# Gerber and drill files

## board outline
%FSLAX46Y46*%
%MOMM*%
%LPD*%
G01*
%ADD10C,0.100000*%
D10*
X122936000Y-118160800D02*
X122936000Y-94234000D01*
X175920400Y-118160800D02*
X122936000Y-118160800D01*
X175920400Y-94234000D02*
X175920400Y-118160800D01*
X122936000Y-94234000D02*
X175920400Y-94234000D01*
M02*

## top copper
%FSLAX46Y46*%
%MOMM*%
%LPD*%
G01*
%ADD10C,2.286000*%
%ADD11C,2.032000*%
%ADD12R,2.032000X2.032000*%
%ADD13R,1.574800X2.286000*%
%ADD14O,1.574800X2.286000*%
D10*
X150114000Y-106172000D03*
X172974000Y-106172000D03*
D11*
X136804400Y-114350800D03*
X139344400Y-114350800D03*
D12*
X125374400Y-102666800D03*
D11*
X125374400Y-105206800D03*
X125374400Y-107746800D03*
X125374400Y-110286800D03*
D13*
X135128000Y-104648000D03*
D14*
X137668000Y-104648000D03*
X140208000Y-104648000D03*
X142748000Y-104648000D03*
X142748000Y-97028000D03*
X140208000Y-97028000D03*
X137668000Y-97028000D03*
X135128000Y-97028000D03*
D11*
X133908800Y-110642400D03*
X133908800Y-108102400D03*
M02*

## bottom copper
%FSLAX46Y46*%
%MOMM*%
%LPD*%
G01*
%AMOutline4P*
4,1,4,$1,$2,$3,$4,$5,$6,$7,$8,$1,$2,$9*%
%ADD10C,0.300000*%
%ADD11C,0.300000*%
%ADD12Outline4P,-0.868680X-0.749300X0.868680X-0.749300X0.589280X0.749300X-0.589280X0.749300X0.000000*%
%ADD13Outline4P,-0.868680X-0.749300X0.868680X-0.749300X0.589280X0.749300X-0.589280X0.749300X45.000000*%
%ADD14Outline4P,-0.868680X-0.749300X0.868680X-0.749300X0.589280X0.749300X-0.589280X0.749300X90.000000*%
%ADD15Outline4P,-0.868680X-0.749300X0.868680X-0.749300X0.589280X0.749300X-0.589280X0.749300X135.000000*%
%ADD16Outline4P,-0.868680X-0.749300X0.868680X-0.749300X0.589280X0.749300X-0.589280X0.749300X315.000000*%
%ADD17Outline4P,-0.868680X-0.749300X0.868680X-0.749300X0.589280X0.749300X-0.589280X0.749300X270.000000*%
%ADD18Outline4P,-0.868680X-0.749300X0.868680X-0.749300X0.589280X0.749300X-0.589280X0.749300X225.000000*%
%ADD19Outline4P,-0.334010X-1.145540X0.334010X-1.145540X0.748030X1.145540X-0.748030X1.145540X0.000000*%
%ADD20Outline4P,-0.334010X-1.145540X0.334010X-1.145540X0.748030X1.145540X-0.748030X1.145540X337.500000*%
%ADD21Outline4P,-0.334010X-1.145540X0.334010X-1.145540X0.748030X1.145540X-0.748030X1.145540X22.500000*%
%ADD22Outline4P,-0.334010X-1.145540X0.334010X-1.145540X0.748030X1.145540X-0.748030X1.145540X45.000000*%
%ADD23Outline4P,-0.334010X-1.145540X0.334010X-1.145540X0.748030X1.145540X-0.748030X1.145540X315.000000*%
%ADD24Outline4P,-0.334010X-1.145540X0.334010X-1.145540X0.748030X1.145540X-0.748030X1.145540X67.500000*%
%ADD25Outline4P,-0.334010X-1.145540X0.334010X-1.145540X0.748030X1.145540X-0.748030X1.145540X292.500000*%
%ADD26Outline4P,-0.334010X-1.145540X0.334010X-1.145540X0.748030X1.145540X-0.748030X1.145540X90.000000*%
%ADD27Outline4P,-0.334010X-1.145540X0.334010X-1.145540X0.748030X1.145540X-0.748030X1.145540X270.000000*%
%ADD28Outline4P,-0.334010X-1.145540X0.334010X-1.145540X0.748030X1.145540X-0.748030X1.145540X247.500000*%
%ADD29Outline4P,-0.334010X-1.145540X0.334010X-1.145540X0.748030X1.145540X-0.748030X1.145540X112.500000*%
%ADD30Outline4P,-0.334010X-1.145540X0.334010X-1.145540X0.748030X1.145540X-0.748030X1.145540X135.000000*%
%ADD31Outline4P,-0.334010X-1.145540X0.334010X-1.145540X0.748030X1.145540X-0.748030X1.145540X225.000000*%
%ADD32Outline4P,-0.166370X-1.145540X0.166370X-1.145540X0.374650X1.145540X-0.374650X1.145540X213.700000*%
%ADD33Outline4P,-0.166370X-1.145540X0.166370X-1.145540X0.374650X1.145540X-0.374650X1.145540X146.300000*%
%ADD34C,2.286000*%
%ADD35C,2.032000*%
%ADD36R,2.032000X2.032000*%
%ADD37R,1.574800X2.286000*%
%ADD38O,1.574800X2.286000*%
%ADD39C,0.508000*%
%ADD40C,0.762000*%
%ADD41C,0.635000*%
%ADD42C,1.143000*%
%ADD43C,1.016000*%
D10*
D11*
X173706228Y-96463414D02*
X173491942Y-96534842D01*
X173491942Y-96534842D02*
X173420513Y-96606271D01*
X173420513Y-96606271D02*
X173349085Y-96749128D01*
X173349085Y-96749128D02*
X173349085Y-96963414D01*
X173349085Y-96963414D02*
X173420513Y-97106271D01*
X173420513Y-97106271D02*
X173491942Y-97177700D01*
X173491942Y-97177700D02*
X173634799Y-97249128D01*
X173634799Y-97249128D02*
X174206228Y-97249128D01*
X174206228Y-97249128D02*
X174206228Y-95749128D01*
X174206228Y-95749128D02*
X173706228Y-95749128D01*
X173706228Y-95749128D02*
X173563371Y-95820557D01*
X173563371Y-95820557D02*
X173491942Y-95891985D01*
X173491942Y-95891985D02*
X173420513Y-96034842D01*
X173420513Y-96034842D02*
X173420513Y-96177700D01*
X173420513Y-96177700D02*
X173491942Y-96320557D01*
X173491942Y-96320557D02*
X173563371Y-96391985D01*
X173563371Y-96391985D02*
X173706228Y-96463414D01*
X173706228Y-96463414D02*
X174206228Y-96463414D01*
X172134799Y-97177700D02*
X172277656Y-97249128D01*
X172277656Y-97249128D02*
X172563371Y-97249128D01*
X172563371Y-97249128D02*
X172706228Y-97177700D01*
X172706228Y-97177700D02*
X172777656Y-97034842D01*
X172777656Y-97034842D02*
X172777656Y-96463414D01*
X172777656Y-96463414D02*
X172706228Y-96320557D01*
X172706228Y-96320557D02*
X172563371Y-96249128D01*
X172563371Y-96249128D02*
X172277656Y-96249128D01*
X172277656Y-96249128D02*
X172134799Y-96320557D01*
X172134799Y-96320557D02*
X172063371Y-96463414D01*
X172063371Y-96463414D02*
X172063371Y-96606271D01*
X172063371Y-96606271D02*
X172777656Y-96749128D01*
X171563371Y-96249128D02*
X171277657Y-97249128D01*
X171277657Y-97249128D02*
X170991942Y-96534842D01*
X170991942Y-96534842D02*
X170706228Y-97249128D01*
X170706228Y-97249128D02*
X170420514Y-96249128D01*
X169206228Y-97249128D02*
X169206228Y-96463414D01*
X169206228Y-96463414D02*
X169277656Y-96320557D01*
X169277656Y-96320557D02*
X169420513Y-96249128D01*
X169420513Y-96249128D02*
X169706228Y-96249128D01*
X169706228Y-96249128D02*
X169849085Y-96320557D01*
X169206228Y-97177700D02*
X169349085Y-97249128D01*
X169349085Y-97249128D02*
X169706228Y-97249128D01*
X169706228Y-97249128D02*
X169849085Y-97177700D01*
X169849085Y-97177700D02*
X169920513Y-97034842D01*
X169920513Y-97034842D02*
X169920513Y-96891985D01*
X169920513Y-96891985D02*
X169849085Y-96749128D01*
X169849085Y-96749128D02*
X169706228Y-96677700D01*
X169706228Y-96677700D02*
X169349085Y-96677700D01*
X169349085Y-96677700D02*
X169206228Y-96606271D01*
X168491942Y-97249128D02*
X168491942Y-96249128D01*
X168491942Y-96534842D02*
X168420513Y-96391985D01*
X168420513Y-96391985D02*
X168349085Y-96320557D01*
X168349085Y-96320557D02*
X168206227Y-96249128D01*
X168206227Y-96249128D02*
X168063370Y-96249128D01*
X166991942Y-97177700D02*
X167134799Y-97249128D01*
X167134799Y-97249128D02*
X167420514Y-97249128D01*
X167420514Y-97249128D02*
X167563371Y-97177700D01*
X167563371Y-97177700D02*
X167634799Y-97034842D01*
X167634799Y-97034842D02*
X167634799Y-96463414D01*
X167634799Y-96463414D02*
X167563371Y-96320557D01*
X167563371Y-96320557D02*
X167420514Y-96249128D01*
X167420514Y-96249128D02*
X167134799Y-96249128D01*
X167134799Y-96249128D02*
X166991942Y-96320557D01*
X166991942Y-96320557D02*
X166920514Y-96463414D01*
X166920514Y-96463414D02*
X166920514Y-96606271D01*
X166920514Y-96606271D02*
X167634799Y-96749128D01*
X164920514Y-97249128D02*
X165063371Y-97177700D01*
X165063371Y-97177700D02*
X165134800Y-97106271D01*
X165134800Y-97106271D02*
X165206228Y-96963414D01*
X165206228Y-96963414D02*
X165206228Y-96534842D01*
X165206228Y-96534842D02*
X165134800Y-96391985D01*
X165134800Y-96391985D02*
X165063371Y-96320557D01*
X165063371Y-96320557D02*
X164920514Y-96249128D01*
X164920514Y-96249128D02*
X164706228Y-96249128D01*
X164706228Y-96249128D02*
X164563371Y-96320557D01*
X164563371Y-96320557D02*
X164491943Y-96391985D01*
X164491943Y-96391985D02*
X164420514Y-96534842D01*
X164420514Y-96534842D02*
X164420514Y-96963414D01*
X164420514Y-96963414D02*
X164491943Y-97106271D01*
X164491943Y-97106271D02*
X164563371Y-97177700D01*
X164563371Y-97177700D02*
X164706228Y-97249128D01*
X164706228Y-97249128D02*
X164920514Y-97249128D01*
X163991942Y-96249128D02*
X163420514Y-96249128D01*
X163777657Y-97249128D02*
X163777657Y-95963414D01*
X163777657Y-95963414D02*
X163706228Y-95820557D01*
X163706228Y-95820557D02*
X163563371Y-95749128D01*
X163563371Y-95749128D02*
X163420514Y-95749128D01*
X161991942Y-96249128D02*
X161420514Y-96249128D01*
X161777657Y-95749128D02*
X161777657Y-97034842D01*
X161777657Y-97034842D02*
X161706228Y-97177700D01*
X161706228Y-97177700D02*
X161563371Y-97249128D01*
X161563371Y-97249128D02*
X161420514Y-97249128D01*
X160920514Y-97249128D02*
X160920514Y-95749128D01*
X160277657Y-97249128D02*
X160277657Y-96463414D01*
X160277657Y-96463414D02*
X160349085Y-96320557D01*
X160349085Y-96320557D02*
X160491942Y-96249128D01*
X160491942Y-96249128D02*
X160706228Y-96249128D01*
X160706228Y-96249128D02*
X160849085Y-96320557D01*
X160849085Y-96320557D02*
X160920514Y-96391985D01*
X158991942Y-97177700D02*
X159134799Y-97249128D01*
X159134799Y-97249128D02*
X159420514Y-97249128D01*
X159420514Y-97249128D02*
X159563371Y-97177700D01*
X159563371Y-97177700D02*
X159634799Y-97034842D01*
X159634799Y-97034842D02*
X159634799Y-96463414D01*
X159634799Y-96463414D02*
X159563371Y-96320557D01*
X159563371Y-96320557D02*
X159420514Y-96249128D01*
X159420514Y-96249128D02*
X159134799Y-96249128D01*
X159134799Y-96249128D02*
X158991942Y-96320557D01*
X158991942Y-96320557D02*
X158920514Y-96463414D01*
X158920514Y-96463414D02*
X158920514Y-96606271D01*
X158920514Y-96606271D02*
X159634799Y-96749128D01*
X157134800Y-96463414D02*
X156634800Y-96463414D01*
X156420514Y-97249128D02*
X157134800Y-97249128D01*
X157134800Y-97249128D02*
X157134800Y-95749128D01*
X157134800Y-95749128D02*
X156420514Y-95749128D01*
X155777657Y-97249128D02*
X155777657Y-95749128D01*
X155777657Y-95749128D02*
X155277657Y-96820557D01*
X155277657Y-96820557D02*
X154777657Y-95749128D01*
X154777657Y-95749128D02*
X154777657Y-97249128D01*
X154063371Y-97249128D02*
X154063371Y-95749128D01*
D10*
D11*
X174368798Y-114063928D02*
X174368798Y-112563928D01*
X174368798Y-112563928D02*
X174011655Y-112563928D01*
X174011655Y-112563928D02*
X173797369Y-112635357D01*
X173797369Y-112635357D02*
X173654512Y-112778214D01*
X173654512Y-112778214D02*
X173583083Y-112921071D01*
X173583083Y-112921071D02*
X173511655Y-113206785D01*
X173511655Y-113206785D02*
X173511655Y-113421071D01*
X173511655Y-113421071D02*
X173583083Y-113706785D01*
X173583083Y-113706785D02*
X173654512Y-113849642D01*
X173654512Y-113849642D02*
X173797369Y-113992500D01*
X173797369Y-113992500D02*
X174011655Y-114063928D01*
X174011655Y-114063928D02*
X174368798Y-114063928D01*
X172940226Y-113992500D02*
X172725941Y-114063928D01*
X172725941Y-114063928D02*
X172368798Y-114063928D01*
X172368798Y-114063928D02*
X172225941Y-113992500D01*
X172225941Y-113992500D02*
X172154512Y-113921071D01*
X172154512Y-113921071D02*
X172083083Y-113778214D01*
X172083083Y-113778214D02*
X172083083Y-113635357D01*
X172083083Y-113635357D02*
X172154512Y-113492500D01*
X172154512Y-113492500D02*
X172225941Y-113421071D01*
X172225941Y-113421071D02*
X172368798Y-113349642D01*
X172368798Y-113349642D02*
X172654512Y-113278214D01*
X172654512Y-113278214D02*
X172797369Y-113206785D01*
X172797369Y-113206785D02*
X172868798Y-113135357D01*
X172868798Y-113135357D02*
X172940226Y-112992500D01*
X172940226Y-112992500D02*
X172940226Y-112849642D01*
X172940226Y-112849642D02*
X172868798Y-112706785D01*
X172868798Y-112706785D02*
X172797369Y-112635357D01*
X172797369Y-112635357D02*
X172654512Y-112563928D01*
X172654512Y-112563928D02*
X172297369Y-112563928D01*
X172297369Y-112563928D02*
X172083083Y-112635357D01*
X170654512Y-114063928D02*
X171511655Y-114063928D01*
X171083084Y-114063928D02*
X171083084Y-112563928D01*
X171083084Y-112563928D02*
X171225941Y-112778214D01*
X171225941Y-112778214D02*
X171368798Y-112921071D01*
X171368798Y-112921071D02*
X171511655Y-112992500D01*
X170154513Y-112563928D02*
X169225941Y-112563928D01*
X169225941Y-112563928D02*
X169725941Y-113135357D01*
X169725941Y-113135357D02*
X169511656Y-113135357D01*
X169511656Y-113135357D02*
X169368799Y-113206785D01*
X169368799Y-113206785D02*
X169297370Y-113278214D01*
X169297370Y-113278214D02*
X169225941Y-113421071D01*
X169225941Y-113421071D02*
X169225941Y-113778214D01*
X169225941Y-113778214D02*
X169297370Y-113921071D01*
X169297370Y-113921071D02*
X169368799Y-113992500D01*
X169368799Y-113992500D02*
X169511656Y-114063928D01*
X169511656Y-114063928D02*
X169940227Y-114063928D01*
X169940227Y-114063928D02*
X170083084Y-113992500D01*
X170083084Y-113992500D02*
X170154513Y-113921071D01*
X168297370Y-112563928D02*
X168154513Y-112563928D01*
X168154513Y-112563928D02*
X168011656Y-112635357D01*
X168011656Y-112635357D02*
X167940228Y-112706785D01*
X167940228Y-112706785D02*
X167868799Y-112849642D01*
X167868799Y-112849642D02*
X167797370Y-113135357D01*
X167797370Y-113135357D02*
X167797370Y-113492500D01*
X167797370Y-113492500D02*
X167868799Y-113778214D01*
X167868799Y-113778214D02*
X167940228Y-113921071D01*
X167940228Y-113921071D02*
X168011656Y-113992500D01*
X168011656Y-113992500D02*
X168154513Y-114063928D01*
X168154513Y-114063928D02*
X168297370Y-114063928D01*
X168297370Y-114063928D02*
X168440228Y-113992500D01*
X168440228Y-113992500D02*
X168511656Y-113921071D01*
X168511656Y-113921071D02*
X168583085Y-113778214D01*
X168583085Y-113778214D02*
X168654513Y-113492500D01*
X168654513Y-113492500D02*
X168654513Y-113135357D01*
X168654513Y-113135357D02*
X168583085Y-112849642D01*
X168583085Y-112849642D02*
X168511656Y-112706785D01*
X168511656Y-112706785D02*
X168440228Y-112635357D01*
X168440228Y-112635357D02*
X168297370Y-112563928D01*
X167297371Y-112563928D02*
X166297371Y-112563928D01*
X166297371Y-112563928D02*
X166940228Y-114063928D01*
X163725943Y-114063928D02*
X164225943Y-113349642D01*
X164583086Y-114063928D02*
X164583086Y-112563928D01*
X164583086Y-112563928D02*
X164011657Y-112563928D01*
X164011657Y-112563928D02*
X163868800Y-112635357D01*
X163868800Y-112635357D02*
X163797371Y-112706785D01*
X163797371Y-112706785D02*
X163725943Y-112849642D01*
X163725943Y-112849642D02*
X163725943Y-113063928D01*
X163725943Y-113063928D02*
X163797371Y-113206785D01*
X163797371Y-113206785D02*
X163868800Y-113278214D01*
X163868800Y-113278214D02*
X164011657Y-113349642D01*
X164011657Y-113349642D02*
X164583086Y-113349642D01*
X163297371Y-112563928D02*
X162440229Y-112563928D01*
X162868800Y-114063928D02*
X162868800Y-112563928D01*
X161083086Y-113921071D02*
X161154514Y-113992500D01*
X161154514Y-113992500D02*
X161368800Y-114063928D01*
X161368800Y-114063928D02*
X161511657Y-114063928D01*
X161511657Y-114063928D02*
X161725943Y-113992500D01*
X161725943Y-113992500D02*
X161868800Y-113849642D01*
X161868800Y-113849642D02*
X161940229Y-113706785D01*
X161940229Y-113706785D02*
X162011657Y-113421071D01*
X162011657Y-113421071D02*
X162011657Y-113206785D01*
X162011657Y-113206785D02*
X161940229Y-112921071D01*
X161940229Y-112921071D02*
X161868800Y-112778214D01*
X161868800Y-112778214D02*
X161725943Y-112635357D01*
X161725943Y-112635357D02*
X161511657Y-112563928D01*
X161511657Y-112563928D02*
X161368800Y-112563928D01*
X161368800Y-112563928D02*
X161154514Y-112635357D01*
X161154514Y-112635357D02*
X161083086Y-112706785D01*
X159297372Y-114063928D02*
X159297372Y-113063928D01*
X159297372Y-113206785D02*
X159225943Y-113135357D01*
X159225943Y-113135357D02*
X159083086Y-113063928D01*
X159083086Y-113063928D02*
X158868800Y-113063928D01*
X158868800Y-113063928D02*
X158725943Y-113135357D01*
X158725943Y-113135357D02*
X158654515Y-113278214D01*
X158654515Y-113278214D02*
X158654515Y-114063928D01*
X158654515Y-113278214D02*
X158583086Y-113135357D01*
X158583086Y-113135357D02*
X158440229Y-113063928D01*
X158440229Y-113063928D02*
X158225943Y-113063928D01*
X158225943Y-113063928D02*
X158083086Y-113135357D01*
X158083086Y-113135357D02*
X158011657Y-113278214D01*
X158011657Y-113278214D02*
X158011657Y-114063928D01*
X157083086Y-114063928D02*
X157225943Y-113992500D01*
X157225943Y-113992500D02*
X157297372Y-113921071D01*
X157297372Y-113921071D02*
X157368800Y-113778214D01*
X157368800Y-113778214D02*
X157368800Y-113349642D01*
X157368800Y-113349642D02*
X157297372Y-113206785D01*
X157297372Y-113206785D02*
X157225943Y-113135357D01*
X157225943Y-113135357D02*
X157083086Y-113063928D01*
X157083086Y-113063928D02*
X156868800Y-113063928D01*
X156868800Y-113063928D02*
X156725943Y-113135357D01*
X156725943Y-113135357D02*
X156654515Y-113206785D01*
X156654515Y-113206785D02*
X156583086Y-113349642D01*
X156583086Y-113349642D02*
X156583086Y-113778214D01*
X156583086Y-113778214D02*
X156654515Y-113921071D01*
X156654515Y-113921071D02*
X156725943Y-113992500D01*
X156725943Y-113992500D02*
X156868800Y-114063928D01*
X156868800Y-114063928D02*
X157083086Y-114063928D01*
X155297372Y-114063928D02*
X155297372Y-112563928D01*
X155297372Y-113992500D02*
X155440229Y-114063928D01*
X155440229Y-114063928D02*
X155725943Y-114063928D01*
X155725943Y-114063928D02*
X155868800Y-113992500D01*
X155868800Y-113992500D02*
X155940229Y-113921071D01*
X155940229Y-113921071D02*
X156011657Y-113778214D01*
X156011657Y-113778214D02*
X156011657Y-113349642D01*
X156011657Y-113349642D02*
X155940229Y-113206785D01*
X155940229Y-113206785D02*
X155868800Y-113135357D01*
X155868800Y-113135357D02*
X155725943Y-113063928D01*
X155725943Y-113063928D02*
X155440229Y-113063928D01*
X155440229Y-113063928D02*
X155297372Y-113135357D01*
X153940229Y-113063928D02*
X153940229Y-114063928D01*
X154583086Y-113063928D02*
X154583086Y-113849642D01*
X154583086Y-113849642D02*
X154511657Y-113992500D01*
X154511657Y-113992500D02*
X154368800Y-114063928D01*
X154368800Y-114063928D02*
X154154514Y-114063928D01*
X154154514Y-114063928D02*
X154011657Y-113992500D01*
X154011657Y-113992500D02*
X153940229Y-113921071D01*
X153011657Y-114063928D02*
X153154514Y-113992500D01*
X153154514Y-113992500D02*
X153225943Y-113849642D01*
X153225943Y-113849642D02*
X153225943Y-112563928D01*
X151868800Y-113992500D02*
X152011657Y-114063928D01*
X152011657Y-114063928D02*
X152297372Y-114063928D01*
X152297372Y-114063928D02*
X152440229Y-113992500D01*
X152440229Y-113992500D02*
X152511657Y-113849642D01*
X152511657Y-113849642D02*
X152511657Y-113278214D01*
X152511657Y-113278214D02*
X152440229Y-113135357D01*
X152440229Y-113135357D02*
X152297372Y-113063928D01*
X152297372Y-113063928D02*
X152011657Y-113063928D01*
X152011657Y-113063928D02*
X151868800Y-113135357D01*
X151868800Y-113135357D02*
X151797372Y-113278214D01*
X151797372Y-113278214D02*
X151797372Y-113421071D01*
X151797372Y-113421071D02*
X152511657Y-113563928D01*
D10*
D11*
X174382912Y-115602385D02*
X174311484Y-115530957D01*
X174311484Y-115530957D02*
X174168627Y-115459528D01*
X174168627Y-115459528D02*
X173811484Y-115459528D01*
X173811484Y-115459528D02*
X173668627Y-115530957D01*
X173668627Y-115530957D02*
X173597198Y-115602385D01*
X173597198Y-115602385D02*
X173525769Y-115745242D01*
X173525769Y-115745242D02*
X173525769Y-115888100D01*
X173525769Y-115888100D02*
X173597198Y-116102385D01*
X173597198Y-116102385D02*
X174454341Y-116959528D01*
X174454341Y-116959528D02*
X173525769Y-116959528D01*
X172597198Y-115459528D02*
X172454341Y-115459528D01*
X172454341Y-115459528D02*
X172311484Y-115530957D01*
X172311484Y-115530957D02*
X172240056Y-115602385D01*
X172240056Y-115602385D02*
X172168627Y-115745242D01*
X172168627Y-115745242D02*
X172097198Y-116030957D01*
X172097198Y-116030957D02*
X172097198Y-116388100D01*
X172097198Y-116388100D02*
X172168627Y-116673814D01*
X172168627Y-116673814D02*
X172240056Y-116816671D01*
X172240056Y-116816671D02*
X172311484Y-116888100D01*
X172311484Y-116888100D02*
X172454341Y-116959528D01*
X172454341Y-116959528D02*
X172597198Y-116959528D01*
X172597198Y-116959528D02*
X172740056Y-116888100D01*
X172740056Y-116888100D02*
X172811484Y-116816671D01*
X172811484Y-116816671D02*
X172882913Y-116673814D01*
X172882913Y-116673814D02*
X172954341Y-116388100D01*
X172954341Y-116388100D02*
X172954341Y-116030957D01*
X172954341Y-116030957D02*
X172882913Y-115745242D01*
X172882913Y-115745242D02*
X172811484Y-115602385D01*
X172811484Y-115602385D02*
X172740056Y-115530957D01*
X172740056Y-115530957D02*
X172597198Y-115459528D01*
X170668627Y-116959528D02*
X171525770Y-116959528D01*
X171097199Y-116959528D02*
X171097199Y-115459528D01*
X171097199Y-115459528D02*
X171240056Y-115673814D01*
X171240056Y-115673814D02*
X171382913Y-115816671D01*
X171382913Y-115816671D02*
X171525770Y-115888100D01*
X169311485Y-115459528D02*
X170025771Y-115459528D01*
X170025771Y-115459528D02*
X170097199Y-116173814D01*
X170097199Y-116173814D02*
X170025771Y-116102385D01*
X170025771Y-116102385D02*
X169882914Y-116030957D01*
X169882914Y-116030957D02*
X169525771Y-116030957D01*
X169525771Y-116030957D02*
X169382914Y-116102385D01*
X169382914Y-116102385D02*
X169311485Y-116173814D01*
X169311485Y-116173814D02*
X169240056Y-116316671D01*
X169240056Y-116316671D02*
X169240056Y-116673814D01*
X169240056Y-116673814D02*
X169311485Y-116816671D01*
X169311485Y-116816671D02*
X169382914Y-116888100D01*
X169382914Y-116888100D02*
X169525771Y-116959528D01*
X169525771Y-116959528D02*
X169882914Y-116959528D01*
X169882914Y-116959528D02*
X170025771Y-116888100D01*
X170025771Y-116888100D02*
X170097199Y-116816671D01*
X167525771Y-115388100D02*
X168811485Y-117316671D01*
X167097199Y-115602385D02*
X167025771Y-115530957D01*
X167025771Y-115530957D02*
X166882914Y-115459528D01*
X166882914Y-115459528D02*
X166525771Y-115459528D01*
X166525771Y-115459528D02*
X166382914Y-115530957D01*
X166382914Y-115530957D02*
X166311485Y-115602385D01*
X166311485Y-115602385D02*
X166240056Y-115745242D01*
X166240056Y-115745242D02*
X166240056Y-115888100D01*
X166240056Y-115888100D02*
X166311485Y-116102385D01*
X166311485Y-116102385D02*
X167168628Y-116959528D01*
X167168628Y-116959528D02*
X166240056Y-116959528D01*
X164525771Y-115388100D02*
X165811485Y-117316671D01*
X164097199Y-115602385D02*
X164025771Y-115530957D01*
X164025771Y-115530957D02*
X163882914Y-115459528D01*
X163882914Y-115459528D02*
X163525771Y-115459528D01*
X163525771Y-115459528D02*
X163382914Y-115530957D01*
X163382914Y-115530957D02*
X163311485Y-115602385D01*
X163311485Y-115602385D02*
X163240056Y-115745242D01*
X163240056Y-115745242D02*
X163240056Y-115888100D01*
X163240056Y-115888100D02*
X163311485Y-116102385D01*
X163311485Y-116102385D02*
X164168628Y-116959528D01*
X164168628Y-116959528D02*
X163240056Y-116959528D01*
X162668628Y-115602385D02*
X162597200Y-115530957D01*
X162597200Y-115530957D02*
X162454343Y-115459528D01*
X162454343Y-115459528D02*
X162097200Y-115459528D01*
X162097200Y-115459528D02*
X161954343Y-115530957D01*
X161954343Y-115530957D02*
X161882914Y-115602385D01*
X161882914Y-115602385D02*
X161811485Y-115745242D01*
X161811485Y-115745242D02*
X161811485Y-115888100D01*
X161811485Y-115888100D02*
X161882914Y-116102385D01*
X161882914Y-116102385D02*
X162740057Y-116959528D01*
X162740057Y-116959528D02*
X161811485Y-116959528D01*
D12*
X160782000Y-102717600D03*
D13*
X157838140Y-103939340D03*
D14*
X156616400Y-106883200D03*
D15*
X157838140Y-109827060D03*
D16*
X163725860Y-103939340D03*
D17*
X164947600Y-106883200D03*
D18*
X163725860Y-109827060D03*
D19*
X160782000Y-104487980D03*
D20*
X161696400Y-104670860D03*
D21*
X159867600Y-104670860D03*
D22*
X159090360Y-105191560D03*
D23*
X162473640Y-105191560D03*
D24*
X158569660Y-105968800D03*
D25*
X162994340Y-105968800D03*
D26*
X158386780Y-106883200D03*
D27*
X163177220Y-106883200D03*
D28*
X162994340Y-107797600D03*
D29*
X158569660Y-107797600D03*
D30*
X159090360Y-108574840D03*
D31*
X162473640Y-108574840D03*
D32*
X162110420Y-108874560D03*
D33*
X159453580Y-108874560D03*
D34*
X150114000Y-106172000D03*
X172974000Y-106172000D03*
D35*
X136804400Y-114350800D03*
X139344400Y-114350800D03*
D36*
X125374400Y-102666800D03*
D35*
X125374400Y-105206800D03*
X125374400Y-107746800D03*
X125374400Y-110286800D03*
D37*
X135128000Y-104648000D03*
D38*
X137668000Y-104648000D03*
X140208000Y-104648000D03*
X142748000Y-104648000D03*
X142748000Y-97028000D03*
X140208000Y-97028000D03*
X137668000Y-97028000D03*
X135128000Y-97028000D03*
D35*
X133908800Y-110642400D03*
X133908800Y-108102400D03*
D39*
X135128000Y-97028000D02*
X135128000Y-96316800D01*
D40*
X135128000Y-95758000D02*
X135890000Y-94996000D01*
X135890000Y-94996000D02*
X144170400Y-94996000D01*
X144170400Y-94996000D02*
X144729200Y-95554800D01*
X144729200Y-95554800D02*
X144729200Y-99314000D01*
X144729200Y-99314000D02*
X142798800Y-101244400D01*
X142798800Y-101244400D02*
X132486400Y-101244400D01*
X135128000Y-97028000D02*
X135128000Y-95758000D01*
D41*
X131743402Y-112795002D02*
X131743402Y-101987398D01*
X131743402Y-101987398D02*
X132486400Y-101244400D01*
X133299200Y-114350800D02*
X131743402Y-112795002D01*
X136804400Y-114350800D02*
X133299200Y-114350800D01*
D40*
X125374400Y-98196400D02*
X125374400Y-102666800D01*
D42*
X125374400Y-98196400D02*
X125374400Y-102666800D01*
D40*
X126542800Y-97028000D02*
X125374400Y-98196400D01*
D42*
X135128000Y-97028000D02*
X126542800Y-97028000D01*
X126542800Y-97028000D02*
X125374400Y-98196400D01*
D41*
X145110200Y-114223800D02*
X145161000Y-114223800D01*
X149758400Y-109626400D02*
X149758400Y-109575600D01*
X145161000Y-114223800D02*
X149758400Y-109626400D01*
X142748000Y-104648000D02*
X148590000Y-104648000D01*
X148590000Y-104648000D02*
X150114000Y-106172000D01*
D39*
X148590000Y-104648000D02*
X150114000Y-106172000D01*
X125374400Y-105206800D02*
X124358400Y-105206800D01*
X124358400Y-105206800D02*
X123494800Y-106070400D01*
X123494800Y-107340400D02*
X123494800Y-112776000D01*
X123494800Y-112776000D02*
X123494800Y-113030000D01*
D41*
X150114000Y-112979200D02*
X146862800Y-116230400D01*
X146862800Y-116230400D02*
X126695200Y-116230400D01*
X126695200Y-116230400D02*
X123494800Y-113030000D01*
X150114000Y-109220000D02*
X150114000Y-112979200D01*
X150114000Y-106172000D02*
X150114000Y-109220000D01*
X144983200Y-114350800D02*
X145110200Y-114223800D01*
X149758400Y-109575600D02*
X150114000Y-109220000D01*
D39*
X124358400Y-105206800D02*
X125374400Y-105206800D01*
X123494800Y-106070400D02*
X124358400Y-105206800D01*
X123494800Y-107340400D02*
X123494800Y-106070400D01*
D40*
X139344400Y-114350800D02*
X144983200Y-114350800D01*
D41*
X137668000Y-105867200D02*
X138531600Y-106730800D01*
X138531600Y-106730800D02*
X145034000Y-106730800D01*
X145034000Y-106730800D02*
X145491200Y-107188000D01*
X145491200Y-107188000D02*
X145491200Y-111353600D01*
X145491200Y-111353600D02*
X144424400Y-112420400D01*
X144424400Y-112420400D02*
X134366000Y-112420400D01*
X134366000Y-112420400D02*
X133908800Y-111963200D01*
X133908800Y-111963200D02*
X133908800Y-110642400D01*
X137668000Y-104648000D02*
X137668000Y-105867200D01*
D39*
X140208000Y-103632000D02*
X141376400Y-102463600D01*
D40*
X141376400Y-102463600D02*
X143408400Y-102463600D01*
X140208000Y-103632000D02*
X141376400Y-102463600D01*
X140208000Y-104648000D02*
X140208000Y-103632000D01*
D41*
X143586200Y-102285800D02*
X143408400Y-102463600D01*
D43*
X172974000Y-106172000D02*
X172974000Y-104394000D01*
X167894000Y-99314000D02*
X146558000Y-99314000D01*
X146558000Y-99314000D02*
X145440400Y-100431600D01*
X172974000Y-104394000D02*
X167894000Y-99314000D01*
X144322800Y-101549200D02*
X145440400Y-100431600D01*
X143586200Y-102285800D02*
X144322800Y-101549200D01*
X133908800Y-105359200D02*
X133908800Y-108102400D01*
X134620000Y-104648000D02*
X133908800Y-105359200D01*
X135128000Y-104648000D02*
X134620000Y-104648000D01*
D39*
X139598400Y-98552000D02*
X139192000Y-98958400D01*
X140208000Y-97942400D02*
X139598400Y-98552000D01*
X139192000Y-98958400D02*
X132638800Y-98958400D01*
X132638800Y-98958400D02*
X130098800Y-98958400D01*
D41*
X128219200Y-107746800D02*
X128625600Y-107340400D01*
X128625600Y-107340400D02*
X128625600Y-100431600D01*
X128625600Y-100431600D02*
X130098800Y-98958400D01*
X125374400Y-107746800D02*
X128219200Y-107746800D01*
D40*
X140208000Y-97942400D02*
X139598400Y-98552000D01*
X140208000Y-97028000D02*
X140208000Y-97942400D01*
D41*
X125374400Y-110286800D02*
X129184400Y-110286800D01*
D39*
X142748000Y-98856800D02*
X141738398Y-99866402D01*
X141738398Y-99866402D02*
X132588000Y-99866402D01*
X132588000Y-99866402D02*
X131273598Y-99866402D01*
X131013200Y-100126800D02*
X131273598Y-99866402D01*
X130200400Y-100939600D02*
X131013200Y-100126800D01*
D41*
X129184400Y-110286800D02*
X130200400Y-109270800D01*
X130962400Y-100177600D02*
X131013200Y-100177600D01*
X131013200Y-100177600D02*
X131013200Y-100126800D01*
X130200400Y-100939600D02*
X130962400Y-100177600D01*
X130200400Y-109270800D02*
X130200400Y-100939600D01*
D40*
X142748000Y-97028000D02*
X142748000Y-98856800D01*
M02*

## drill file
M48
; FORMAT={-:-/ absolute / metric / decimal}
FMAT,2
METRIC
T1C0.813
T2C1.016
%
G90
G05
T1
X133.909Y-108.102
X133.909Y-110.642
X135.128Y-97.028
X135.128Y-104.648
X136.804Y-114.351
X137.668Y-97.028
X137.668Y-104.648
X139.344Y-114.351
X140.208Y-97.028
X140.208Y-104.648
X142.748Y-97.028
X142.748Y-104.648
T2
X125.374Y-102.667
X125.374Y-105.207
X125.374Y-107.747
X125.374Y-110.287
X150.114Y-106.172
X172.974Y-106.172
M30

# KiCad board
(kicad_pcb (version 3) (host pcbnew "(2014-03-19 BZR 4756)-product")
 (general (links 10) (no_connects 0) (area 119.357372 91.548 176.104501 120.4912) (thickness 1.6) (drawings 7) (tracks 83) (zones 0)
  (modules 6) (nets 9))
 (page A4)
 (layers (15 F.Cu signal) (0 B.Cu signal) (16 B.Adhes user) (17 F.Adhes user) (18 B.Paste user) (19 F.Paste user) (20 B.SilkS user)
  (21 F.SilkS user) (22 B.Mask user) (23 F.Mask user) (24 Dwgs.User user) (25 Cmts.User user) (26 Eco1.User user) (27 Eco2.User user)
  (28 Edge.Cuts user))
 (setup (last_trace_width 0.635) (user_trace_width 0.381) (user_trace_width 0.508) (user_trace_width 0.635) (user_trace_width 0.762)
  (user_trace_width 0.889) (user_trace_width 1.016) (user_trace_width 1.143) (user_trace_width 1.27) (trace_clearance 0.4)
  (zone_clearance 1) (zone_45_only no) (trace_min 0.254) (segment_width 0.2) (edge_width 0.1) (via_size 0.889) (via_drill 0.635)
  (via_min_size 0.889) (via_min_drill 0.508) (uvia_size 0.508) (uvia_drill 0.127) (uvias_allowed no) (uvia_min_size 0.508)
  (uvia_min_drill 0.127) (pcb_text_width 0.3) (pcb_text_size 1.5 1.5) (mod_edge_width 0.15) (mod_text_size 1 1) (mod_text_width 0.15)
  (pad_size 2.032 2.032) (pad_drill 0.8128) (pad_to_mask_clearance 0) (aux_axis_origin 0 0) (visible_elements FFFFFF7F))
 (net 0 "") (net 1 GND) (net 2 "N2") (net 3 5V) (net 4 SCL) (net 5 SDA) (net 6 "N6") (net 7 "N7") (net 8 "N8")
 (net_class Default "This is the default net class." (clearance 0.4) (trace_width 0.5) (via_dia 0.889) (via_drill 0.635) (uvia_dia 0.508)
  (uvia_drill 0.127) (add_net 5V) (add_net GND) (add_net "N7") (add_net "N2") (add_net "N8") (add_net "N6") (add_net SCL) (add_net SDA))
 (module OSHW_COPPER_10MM (layer B.Cu) (at 160.782 106.8832 180)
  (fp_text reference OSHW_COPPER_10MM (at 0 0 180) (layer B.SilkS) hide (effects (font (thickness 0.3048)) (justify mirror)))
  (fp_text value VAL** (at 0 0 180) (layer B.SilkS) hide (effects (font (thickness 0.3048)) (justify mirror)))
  (pad "" smd trapezoid (at 0 4.1656) (size 1.45796 1.4986) (rect_delta 0 0.2794) (layers B.Cu B.Paste B.Mask))
  (pad "" smd trapezoid (at 2.94386 2.94386 45) (size 1.45796 1.4986) (rect_delta 0 0.2794) (layers B.Cu B.Paste B.Mask))
  (pad "" smd trapezoid (at 4.1656 0 90) (size 1.45796 1.4986) (rect_delta 0 0.2794) (layers B.Cu B.Paste B.Mask))
  (pad "" smd trapezoid (at 2.94386 -2.94386 135) (size 1.45796 1.4986) (rect_delta 0 0.2794) (layers B.Cu B.Paste B.Mask))
  (pad "" smd trapezoid (at -2.94386 2.94386 315) (size 1.45796 1.4986) (rect_delta 0 0.2794) (layers B.Cu B.Paste B.Mask))
  (pad "" smd trapezoid (at -4.1656 0 270) (size 1.45796 1.4986) (rect_delta 0 0.2794) (layers B.Cu B.Paste B.Mask))
  (pad "" smd trapezoid (at -2.94386 -2.94386 225) (size 1.45796 1.4986) (rect_delta 0 0.2794) (layers B.Cu B.Paste B.Mask))
  (pad "" smd trapezoid (at 0 2.39522) (size 1.08204 2.29108) (rect_delta 0 -0.41402) (layers B.Cu B.Paste B.Mask))
  (pad "" smd trapezoid (at -0.9144 2.21234 337.5) (size 1.08204 2.29108) (rect_delta 0 -0.41402) (layers B.Cu B.Paste B.Mask))
  (pad "" smd trapezoid (at 0.9144 2.21234 22.5) (size 1.08204 2.29108) (rect_delta 0 -0.41402) (layers B.Cu B.Paste B.Mask))
  (pad "" smd trapezoid (at 1.69164 1.69164 45) (size 1.08204 2.29108) (rect_delta 0 -0.41402) (layers B.Cu B.Paste B.Mask))
  (pad "" smd trapezoid (at -1.69164 1.69164 315) (size 1.08204 2.29108) (rect_delta 0 -0.41402) (layers B.Cu B.Paste B.Mask))
  (pad "" smd trapezoid (at 2.21234 0.9144 67.5) (size 1.08204 2.29108) (rect_delta 0 -0.41402) (layers B.Cu B.Paste B.Mask))
  (pad "" smd trapezoid (at -2.21234 0.9144 292.5) (size 1.08204 2.29108) (rect_delta 0 -0.41402) (layers B.Cu B.Paste B.Mask))
  (pad "" smd trapezoid (at 2.39522 0 90) (size 1.08204 2.29108) (rect_delta 0 -0.41402) (layers B.Cu B.Paste B.Mask))
  (pad "" smd trapezoid (at -2.39522 0 270) (size 1.08204 2.29108) (rect_delta 0 -0.41402) (layers B.Cu B.Paste B.Mask))
  (pad "" smd trapezoid (at -2.21234 -0.9144 247.5) (size 1.08204 2.29108) (rect_delta 0 -0.41402) (layers B.Cu B.Paste B.Mask))
  (pad "" smd trapezoid (at 2.21234 -0.9144 112.5) (size 1.08204 2.29108) (rect_delta 0 -0.41402) (layers B.Cu B.Paste B.Mask))
  (pad "" smd trapezoid (at 1.69164 -1.69164 135) (size 1.08204 2.29108) (rect_delta 0 -0.41402) (layers B.Cu B.Paste B.Mask))
  (pad "" smd trapezoid (at -1.69164 -1.69164 225) (size 1.08204 2.29108) (rect_delta 0 -0.41402) (layers B.Cu B.Paste B.Mask))
  (pad "" smd trapezoid (at -1.32842 -1.99136 213.7) (size 0.54102 2.29108) (rect_delta 0 -0.20828) (layers B.Cu B.Paste B.Mask))
  (pad "" smd trapezoid (at 1.32842 -1.99136 146.3) (size 0.54102 2.29108) (rect_delta 0 -0.20828) (layers B.Cu B.Paste B.Mask)))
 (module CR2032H (layer F.Cu) (at 157.734 106.172)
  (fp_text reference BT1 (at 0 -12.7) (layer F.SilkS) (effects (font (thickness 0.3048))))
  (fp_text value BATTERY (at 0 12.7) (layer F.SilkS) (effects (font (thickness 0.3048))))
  (pad 2 thru_hole circle (at -7.62 0) (size 2.286 2.286) (drill 1.016) (layers *.Cu *.Mask F.SilkS) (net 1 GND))
  (pad 1 thru_hole circle (at 15.24 0) (size 2.286 2.286) (drill 1.016) (layers *.Cu *.Mask F.SilkS) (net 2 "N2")))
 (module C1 (layer F.Cu) (at 138.0744 114.3508)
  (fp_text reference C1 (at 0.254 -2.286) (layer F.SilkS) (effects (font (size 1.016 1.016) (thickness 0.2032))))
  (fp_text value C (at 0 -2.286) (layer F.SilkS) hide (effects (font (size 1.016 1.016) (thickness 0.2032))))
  (pad 1 thru_hole circle (at -1.27 0) (size 2.032 2.032) (drill 0.8128) (layers *.Cu *.Mask F.SilkS) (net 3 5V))
  (pad 2 thru_hole circle (at 1.27 0) (size 2.032 2.032) (drill 0.8128) (layers *.Cu *.Mask F.SilkS) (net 1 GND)))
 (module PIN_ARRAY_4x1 (layer F.Cu) (at 125.3744 106.4768 270)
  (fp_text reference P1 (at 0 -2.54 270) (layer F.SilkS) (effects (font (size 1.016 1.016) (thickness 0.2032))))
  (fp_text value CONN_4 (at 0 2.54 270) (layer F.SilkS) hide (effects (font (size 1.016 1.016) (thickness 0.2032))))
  (pad 1 thru_hole rect (at -3.81 0 270) (size 2.032 2.032) (drill 1.016) (layers *.Cu *.Mask F.SilkS) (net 3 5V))
  (pad 2 thru_hole circle (at -1.27 0 270) (size 2.032 2.032) (drill 1.016) (layers *.Cu *.Mask F.SilkS) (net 1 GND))
  (pad 3 thru_hole circle (at 1.27 0 270) (size 2.032 2.032) (drill 1.016) (layers *.Cu *.Mask F.SilkS) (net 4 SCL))
  (pad 4 thru_hole circle (at 3.81 0 270) (size 2.032 2.032) (drill 1.016) (layers *.Cu *.Mask F.SilkS) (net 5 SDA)))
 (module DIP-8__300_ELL (layer F.Cu) (at 138.938 100.838)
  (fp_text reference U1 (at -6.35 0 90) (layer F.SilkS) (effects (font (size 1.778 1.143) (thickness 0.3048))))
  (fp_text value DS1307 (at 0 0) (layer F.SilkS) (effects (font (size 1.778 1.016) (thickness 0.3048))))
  (pad 1 thru_hole rect (at -3.81 3.81) (size 1.5748 2.286) (drill 0.8128) (layers *.Cu *.Mask F.SilkS) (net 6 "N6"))
  (pad 2 thru_hole oval (at -1.27 3.81) (size 1.5748 2.286) (drill 0.8128) (layers *.Cu *.Mask F.SilkS) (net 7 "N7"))
  (pad 3 thru_hole oval (at 1.27 3.81) (size 1.5748 2.286) (drill 0.8128) (layers *.Cu *.Mask F.SilkS) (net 2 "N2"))
  (pad 4 thru_hole oval (at 3.81 3.81) (size 1.5748 2.286) (drill 0.8128) (layers *.Cu *.Mask F.SilkS) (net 1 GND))
  (pad 5 thru_hole oval (at 3.81 -3.81) (size 1.5748 2.286) (drill 0.8128) (layers *.Cu *.Mask F.SilkS) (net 5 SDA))
  (pad 6 thru_hole oval (at 1.27 -3.81) (size 1.5748 2.286) (drill 0.8128) (layers *.Cu *.Mask F.SilkS) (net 4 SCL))
  (pad 7 thru_hole oval (at -1.27 -3.81) (size 1.5748 2.286) (drill 0.8128) (layers *.Cu *.Mask F.SilkS) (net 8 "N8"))
  (pad 8 thru_hole oval (at -3.81 -3.81) (size 1.5748 2.286) (drill 0.8128) (layers *.Cu *.Mask F.SilkS) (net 3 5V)))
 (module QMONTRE (layer F.Cu) (at 133.9088 109.3724 90)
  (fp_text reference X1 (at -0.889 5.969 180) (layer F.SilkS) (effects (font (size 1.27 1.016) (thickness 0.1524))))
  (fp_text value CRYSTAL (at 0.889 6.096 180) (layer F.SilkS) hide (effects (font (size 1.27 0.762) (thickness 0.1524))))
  (pad 1 thru_hole circle (at -1.27 0 90) (size 2.032 2.032) (drill 0.8128) (layers *.Cu *.Mask F.SilkS) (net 7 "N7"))
  (pad 2 thru_hole circle (at 1.27 0 90) (size 2.032 2.032) (drill 0.8128) (layers *.Cu *.Mask F.SilkS) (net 6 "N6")))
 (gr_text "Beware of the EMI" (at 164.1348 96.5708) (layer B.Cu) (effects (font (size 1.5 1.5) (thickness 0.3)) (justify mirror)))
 (gr_line (start 122.936 118.1608) (end 122.936 94.234) (angle 90) (layer Edge.Cuts) (width 0.1))
 (gr_line (start 175.9204 118.1608) (end 122.936 118.1608) (angle 90) (layer Edge.Cuts) (width 0.1))
 (gr_line (start 175.9204 94.234) (end 175.9204 118.1608) (angle 90) (layer Edge.Cuts) (width 0.1))
 (gr_line (start 122.936 94.234) (end 175.9204 94.234) (angle 90) (layer Edge.Cuts) (width 0.1))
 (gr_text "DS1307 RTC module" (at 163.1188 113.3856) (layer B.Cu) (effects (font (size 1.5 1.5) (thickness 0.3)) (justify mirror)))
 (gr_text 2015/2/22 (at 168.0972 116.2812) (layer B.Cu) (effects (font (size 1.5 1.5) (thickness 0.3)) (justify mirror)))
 (segment (start 135.128 97.028) (end 135.128 96.3168) (width 0.508) (layer B.Cu) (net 3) (status 30))
 (segment (start 135.128 95.758) (end 135.89 94.996) (width 0.762) (layer B.Cu) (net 3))
 (segment (start 135.89 94.996) (end 144.1704 94.996) (width 0.762) (layer B.Cu) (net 3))
 (segment (start 144.1704 94.996) (end 144.7292 95.5548) (width 0.762) (layer B.Cu) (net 3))
 (segment (start 144.7292 95.5548) (end 144.7292 99.314) (width 0.762) (layer B.Cu) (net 3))
 (segment (start 144.7292 99.314) (end 142.7988 101.2444) (width 0.762) (layer B.Cu) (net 3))
 (segment (start 142.7988 101.2444) (end 132.4864 101.2444) (width 0.762) (layer B.Cu) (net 3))
 (segment (start 135.128 97.028) (end 135.128 95.758) (width 0.762) (layer B.Cu) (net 3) (status 10))
 (segment (start 131.743402 112.795002) (end 131.743402 101.987398) (width 0.635) (layer B.Cu) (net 3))
 (segment (start 131.743402 101.987398) (end 132.4864 101.2444) (width 0.635) (layer B.Cu) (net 3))
 (segment (start 133.2992 114.3508) (end 131.743402 112.795002) (width 0.635) (layer B.Cu) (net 3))
 (segment (start 136.8044 114.3508) (end 133.2992 114.3508) (width 0.635) (layer B.Cu) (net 3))
 (segment (start 125.3744 98.1964) (end 125.3744 102.6668) (width 0.762) (layer B.Cu) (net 3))
 (segment (start 125.3744 98.1964) (end 125.3744 102.6668) (width 1.143) (layer B.Cu) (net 3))
 (segment (start 126.5428 97.028) (end 125.3744 98.1964) (width 0.762) (layer B.Cu) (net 3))
 (segment (start 135.128 97.028) (end 126.5428 97.028) (width 1.143) (layer B.Cu) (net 3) (status 10))
 (segment (start 126.5428 97.028) (end 125.3744 98.1964) (width 1.143) (layer B.Cu) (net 3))
 (segment (start 145.1102 114.2238) (end 145.161 114.2238) (width 0.635) (layer B.Cu) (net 1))
 (segment (start 149.7584 109.6264) (end 149.7584 109.5756) (width 0.635) (layer B.Cu) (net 1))
 (segment (start 145.161 114.2238) (end 149.7584 109.6264) (width 0.635) (layer B.Cu) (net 1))
 (segment (start 142.748 104.648) (end 148.59 104.648) (width 0.635) (layer B.Cu) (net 1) (status 400000))
 (segment (start 148.59 104.648) (end 150.114 106.172) (width 0.635) (layer B.Cu) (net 1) (status 800000))
 (segment (start 148.59 104.648) (end 150.114 106.172) (width 0.508) (layer B.Cu) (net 1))
 (segment (start 125.3744 105.2068) (end 124.3584 105.2068) (width 0.508) (layer B.Cu) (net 1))
 (segment (start 124.3584 105.2068) (end 123.4948 106.0704) (width 0.508) (layer B.Cu) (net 1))
 (segment (start 123.4948 107.3404) (end 123.4948 112.776) (width 0.508) (layer B.Cu) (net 1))
 (segment (start 123.4948 112.776) (end 123.4948 113.03) (width 0.508) (layer B.Cu) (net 1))
 (segment (start 150.114 112.9792) (end 146.8628 116.2304) (width 0.635) (layer B.Cu) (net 1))
 (segment (start 146.8628 116.2304) (end 126.6952 116.2304) (width 0.635) (layer B.Cu) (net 1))
 (segment (start 126.6952 116.2304) (end 123.4948 113.03) (width 0.635) (layer B.Cu) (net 1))
 (segment (start 150.114 109.22) (end 150.114 112.9792) (width 0.635) (layer B.Cu) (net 1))
 (segment (start 150.114 106.172) (end 150.114 109.22) (width 0.635) (layer B.Cu) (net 1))
 (segment (start 144.9832 114.3508) (end 145.1102 114.2238) (width 0.635) (layer B.Cu) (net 1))
 (segment (start 149.7584 109.5756) (end 150.114 109.22) (width 0.635) (layer B.Cu) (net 1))
 (segment (start 124.3584 105.2068) (end 125.3744 105.2068) (width 0.508) (layer B.Cu) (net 1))
 (segment (start 123.4948 106.0704) (end 124.3584 105.2068) (width 0.508) (layer B.Cu) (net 1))
 (segment (start 123.4948 107.3404) (end 123.4948 106.0704) (width 0.508) (layer B.Cu) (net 1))
 (segment (start 139.3444 114.3508) (end 144.9832 114.3508) (width 0.762) (layer B.Cu) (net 1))
 (segment (start 137.668 105.8672) (end 138.5316 106.7308) (width 0.635) (layer B.Cu) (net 7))
 (segment (start 138.5316 106.7308) (end 145.034 106.7308) (width 0.635) (layer B.Cu) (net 7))
 (segment (start 145.034 106.7308) (end 145.4912 107.188) (width 0.635) (layer B.Cu) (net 7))
 (segment (start 145.4912 107.188) (end 145.4912 111.3536) (width 0.635) (layer B.Cu) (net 7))
 (segment (start 145.4912 111.3536) (end 144.4244 112.4204) (width 0.635) (layer B.Cu) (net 7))
 (segment (start 144.4244 112.4204) (end 134.366 112.4204) (width 0.635) (layer B.Cu) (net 7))
 (segment (start 134.366 112.4204) (end 133.9088 111.9632) (width 0.635) (layer B.Cu) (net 7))
 (segment (start 133.9088 111.9632) (end 133.9088 110.6424) (width 0.635) (layer B.Cu) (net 7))
 (segment (start 137.668 104.648) (end 137.668 105.8672) (width 0.635) (layer B.Cu) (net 7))
 (segment (start 140.208 103.632) (end 141.3764 102.4636) (width 0.508) (layer B.Cu) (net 2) (status 10))
 (segment (start 141.3764 102.4636) (end 143.4084 102.4636) (width 0.762) (layer B.Cu) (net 2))
 (segment (start 140.208 103.632) (end 141.3764 102.4636) (width 0.762) (layer B.Cu) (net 2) (status 10))
 (segment (start 140.208 104.648) (end 140.208 103.632) (width 0.762) (layer B.Cu) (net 2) (status 30))
 (segment (start 143.5862 102.2858) (end 143.4084 102.4636) (width 0.635) (layer B.Cu) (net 2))
 (segment (start 172.974 106.172) (end 172.974 104.394) (width 1.016) (layer B.Cu) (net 2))
 (segment (start 167.894 99.314) (end 146.558 99.314) (width 1.016) (layer B.Cu) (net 2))
 (segment (start 146.558 99.314) (end 145.4404 100.4316) (width 1.016) (layer B.Cu) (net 2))
 (segment (start 172.974 104.394) (end 167.894 99.314) (width 1.016) (layer B.Cu) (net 2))
 (segment (start 144.3228 101.5492) (end 145.4404 100.4316) (width 1.016) (layer B.Cu) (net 2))
 (segment (start 143.5862 102.2858) (end 144.3228 101.5492) (width 1.016) (layer B.Cu) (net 2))
 (segment (start 133.9088 105.3592) (end 133.9088 108.1024) (width 1.016) (layer B.Cu) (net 6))
 (segment (start 134.62 104.648) (end 133.9088 105.3592) (width 1.016) (layer B.Cu) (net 6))
 (segment (start 135.128 104.648) (end 134.62 104.648) (width 1.016) (layer B.Cu) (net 6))
 (segment (start 139.5984 98.552) (end 139.192 98.9584) (width 0.508) (layer B.Cu) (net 4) (status 10))
 (segment (start 140.208 97.9424) (end 139.5984 98.552) (width 0.508) (layer B.Cu) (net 4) (status 10))
 (segment (start 139.192 98.9584) (end 132.6388 98.9584) (width 0.508) (layer B.Cu) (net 4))
 (segment (start 132.6388 98.9584) (end 130.0988 98.9584) (width 0.508) (layer B.Cu) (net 4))
 (segment (start 128.2192 107.7468) (end 128.6256 107.3404) (width 0.635) (layer B.Cu) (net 4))
 (segment (start 128.6256 107.3404) (end 128.6256 100.4316) (width 0.635) (layer B.Cu) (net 4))
 (segment (start 128.6256 100.4316) (end 130.0988 98.9584) (width 0.635) (layer B.Cu) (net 4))
 (segment (start 125.3744 107.7468) (end 128.2192 107.7468) (width 0.635) (layer B.Cu) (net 4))
 (segment (start 140.208 97.9424) (end 139.5984 98.552) (width 0.762) (layer B.Cu) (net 4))
 (segment (start 140.208 97.028) (end 140.208 97.9424) (width 0.762) (layer B.Cu) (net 4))
 (segment (start 125.3744 110.2868) (end 129.1844 110.2868) (width 0.635) (layer B.Cu) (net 5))
 (segment (start 142.748 98.8568) (end 141.738398 99.866402) (width 0.508) (layer B.Cu) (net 5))
 (segment (start 141.738398 99.866402) (end 132.588 99.866402) (width 0.508) (layer B.Cu) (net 5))
 (segment (start 132.588 99.866402) (end 131.273598 99.866402) (width 0.508) (layer B.Cu) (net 5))
 (segment (start 131.0132 100.1268) (end 131.273598 99.866402) (width 0.508) (layer B.Cu) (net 5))
 (segment (start 130.2004 100.9396) (end 131.0132 100.1268) (width 0.508) (layer B.Cu) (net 5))
 (segment (start 129.1844 110.2868) (end 130.2004 109.2708) (width 0.635) (layer B.Cu) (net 5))
 (segment (start 130.9624 100.1776) (end 131.0132 100.1776) (width 0.635) (layer B.Cu) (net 5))
 (segment (start 131.0132 100.1776) (end 131.0132 100.1268) (width 0.635) (layer B.Cu) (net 5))
 (segment (start 130.2004 100.9396) (end 130.9624 100.1776) (width 0.635) (layer B.Cu) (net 5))
 (segment (start 130.2004 109.2708) (end 130.2004 100.9396) (width 0.635) (layer B.Cu) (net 5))
 (segment (start 142.748 97.028) (end 142.748 98.8568) (width 0.762) (layer B.Cu) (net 5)))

